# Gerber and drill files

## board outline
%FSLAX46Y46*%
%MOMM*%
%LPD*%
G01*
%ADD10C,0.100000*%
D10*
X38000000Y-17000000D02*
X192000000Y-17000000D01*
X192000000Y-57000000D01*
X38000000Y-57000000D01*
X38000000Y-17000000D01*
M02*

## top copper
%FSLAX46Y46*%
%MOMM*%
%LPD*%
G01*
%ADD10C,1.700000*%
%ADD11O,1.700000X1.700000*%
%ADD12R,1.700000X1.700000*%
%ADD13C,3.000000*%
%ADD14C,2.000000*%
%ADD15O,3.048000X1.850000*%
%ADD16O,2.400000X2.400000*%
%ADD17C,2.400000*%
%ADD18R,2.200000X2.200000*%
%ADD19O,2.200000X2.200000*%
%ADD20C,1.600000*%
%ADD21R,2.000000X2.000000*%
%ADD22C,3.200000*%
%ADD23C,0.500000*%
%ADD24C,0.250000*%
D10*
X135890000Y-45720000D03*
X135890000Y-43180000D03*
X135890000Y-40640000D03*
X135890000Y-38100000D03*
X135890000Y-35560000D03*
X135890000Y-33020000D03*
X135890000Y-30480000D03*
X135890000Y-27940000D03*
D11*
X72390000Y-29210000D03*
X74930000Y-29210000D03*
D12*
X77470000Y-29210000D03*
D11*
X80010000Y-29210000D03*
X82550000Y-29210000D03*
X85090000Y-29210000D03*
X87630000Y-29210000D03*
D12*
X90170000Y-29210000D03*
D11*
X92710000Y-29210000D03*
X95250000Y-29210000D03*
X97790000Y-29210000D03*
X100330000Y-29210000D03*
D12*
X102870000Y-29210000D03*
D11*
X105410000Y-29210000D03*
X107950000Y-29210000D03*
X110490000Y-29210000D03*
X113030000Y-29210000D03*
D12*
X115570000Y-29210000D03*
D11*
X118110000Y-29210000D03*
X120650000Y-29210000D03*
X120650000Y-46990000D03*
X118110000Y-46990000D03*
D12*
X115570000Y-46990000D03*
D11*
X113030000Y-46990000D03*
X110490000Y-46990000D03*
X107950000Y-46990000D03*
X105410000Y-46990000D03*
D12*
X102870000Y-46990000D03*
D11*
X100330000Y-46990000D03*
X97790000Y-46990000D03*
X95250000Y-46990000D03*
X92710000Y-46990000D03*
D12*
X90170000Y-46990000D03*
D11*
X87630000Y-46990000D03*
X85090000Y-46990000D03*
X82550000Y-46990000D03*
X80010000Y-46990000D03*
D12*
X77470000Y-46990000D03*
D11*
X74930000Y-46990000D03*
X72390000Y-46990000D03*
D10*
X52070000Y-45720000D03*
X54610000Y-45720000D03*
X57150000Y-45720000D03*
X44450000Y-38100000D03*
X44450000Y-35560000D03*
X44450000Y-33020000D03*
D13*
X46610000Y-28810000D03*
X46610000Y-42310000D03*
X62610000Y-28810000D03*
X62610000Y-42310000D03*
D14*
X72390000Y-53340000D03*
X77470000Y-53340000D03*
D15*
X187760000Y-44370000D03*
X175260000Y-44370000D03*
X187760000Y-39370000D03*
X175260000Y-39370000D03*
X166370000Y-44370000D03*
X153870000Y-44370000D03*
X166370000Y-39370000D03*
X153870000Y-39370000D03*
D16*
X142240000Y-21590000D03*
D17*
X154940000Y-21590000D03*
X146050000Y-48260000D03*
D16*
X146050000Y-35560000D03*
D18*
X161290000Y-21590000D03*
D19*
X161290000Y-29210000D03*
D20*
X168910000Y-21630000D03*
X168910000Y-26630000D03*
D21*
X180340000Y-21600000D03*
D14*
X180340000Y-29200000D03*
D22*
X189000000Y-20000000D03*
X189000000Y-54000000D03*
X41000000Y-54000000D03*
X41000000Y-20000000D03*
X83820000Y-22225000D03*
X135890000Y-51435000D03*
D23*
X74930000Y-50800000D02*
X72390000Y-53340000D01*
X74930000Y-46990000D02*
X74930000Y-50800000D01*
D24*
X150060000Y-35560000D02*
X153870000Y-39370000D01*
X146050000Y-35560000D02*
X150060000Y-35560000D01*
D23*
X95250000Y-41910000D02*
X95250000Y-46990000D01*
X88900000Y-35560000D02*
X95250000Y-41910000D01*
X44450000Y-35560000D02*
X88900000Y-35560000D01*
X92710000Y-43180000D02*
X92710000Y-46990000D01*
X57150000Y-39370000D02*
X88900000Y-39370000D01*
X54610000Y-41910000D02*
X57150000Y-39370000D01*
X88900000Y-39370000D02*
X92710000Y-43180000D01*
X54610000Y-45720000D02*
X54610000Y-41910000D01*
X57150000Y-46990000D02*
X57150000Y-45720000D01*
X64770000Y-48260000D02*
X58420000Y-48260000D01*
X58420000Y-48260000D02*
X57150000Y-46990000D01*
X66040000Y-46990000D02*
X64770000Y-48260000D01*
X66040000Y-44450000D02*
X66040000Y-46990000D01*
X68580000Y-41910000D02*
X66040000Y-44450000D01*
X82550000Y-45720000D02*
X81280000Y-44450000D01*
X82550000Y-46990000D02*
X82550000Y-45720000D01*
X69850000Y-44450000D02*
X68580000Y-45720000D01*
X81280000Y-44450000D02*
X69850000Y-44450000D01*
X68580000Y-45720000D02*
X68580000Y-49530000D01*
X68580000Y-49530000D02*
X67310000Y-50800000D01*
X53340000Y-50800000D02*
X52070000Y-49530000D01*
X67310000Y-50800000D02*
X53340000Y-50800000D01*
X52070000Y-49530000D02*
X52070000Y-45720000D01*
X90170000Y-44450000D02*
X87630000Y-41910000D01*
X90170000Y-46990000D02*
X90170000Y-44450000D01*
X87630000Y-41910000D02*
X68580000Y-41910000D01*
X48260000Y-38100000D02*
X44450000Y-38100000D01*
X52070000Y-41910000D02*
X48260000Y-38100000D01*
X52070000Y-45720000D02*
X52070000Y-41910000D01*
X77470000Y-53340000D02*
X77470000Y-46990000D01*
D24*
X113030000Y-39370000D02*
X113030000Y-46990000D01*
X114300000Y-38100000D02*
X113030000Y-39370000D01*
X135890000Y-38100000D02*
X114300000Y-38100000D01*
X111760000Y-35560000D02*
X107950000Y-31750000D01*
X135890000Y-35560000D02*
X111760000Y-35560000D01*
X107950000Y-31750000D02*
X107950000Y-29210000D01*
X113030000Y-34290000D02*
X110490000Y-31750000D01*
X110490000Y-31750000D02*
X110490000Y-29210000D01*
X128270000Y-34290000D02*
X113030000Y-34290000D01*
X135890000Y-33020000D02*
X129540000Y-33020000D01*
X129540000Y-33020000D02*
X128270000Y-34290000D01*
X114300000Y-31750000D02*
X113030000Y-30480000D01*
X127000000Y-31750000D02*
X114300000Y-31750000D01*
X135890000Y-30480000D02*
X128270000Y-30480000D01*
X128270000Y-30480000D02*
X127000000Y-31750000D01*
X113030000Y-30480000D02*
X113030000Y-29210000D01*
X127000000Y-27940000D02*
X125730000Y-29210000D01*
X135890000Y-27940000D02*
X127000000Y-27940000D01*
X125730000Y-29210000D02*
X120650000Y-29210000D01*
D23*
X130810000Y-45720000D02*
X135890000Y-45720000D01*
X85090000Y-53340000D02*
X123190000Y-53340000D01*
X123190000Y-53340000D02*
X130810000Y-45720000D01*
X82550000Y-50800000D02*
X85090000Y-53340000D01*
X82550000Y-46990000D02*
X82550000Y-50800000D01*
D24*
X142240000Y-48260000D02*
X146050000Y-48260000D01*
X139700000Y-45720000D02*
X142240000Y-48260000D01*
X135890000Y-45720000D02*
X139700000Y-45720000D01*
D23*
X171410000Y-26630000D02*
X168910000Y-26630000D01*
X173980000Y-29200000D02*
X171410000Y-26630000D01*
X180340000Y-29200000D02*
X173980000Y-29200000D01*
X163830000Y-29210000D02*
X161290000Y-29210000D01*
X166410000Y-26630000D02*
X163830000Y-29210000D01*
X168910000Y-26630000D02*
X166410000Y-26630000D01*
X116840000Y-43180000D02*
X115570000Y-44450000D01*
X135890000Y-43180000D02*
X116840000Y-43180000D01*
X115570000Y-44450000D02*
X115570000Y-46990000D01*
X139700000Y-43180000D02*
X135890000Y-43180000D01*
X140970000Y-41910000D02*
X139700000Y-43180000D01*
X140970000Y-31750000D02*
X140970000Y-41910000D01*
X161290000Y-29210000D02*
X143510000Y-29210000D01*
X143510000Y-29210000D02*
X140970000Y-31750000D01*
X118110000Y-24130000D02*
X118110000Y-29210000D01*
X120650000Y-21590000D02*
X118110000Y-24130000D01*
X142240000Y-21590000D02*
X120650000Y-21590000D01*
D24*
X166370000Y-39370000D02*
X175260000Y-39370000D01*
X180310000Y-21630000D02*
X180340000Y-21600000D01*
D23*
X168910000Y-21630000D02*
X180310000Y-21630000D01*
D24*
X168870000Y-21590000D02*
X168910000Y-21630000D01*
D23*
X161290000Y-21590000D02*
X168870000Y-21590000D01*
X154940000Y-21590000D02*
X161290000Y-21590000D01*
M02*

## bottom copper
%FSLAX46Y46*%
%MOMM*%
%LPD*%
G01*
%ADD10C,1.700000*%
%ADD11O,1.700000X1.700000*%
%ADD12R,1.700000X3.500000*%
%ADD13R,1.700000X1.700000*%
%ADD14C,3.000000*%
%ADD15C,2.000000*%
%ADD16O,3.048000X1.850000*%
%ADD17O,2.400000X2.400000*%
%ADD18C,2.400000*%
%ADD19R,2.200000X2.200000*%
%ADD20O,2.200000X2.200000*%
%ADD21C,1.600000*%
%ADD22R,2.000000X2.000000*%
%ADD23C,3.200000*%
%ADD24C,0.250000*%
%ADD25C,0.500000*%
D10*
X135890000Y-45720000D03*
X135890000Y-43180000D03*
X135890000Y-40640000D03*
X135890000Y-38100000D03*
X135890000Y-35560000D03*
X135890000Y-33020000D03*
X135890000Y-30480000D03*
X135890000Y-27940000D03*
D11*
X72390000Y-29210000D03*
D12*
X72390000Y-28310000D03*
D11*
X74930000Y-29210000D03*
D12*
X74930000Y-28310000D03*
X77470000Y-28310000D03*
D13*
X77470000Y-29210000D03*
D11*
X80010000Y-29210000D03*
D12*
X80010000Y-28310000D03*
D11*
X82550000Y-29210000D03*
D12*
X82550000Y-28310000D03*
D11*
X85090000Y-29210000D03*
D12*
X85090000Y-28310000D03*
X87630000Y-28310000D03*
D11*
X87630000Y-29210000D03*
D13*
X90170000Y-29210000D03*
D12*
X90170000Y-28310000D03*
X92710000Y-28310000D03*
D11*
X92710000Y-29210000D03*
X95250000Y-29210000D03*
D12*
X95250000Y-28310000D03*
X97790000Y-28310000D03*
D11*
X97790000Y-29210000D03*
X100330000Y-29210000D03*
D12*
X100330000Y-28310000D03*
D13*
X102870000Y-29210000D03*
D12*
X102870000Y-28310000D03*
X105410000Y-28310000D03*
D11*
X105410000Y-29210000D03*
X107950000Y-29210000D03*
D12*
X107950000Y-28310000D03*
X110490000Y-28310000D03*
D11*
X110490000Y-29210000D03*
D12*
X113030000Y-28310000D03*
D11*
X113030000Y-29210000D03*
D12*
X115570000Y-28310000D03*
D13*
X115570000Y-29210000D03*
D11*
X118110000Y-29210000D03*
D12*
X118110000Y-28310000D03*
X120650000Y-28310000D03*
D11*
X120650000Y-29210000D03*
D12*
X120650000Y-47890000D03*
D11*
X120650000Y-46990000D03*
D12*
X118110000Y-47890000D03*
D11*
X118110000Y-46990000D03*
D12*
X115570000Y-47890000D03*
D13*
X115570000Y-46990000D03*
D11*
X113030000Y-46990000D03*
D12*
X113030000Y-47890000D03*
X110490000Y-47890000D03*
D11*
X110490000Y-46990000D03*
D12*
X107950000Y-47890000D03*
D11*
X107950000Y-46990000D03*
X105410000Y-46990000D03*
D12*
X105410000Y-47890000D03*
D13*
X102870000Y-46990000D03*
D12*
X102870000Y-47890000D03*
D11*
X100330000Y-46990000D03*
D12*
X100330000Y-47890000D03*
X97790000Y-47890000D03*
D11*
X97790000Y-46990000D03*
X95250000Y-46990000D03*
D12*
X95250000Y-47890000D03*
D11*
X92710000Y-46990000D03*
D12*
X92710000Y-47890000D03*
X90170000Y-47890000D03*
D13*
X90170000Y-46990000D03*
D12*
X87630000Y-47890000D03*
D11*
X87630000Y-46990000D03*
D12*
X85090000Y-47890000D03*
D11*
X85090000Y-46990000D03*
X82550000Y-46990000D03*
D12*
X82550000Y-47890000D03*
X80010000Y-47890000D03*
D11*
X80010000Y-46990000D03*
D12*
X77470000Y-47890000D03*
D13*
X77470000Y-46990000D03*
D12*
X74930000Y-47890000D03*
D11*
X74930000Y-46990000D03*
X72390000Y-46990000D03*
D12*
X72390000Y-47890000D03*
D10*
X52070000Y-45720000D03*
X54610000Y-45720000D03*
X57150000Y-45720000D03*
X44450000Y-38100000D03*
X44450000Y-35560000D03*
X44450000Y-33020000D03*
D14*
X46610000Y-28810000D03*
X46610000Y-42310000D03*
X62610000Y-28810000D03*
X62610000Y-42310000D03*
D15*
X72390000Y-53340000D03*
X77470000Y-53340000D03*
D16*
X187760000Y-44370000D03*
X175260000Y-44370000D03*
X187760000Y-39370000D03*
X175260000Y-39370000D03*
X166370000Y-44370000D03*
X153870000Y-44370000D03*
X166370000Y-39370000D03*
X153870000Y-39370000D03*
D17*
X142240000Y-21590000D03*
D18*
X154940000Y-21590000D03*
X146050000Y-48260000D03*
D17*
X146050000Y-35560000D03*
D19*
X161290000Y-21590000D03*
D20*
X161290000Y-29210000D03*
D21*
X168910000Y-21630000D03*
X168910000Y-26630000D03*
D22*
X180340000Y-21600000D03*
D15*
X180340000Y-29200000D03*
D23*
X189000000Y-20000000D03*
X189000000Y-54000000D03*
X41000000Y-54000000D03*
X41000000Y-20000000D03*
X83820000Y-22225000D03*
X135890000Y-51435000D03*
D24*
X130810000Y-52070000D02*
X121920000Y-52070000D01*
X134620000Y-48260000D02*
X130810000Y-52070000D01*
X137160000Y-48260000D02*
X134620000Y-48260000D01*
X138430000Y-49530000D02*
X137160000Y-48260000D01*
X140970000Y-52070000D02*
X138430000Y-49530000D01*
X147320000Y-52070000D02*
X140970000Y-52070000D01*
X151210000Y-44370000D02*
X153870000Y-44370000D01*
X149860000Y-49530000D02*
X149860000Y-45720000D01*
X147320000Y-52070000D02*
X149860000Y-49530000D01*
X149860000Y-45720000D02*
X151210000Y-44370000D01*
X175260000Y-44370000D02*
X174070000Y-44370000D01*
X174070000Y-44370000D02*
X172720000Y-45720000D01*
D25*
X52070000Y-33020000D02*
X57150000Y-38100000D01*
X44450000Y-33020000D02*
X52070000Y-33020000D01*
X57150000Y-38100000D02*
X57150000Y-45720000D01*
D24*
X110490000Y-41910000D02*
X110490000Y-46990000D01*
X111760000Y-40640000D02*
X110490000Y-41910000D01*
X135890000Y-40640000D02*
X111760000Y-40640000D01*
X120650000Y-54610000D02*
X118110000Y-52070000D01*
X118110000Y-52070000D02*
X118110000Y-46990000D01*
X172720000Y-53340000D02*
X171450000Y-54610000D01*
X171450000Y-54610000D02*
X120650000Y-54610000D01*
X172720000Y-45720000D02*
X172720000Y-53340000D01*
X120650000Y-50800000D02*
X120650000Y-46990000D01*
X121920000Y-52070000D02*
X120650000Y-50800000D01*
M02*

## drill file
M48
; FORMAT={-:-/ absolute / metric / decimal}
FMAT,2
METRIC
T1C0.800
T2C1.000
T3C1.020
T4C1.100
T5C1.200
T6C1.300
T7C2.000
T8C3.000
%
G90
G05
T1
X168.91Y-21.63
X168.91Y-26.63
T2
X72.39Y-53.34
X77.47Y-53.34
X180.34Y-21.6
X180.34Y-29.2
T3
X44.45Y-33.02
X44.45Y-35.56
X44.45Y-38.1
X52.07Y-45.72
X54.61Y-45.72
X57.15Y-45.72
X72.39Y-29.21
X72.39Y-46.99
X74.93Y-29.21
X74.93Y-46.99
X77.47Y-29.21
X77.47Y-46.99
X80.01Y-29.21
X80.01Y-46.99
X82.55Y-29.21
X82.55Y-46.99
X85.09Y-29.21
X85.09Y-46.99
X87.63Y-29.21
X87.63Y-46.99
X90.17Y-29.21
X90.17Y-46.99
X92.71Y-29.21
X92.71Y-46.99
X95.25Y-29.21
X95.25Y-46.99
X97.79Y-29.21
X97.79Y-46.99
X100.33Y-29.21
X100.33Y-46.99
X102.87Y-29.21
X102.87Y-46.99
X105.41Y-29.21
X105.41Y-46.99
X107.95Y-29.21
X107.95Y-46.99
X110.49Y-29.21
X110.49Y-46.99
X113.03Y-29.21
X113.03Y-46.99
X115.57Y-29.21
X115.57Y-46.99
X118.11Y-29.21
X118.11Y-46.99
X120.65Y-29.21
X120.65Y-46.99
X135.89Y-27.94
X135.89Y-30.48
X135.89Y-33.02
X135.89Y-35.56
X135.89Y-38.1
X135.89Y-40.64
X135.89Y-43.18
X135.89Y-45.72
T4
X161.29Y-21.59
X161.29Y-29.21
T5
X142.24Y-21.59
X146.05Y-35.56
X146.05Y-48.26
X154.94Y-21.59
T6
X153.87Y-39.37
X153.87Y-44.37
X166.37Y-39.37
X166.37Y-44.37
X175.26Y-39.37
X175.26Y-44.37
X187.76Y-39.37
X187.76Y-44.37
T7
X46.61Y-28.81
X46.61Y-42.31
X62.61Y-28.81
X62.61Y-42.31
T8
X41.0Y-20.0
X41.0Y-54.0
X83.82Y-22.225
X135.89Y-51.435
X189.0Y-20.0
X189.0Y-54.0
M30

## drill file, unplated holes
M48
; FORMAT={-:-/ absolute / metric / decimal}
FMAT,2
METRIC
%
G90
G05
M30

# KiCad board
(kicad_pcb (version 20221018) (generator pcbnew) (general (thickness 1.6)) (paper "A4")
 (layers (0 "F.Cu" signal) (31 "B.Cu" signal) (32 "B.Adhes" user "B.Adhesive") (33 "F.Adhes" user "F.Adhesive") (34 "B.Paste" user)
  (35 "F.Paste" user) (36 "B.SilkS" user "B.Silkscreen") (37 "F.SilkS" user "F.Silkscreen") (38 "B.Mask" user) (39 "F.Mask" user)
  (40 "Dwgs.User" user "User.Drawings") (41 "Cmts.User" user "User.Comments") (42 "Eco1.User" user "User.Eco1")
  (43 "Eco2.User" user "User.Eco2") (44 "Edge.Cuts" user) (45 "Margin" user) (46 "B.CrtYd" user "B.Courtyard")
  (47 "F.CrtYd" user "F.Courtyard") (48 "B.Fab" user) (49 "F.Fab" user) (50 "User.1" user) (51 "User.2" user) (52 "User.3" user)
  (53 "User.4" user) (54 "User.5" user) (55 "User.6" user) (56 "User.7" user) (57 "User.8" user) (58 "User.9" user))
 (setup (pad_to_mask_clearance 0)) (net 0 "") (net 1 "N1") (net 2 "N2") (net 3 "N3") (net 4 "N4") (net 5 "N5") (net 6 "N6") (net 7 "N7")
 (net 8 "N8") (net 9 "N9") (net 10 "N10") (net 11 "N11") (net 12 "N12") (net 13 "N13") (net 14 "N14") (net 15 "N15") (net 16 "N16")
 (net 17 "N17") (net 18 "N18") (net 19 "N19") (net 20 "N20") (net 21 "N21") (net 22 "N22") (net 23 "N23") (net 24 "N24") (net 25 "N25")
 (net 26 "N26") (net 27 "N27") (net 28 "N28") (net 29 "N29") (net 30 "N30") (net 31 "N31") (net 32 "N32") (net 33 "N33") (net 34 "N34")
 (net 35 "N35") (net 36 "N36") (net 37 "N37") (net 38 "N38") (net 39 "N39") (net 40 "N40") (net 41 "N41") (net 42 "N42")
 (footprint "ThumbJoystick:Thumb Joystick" (layer "F.Cu") (at 54.61 35.56)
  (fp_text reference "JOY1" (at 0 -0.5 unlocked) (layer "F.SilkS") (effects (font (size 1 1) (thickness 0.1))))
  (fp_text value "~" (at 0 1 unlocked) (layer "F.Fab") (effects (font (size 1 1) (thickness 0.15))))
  (pad "1" thru_hole circle (at -2.54 10.16) (size 1.7 1.7) (drill 1.02) (layers "*.Cu" "*.Mask") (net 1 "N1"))
  (pad "2" thru_hole circle (at 0 10.16) (size 1.7 1.7) (drill 1.02) (layers "*.Cu" "*.Mask") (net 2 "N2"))
  (pad "3" thru_hole circle (at 2.54 10.16) (size 1.7 1.7) (drill 1.02) (layers "*.Cu" "*.Mask") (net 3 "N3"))
  (pad "4" thru_hole circle (at -10.16 2.54) (size 1.7 1.7) (drill 1.02) (layers "*.Cu" "*.Mask") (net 1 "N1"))
  (pad "5" thru_hole circle (at -10.16 0) (size 1.7 1.7) (drill 1.02) (layers "*.Cu" "*.Mask") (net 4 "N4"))
  (pad "6" thru_hole circle (at -10.16 -2.54) (size 1.7 1.7) (drill 1.02) (layers "*.Cu" "*.Mask") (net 3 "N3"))
  (pad "8" thru_hole circle (at -8 -6.75) (size 3 3) (drill 2) (layers "*.Cu" "*.Mask"))
  (pad "8" thru_hole circle (at -8 6.75) (size 3 3) (drill 2) (layers "*.Cu" "*.Mask"))
  (pad "8" thru_hole circle (at 8 -6.75) (size 3 3) (drill 2) (layers "*.Cu" "*.Mask"))
  (pad "8" thru_hole circle (at 8 6.75) (size 3 3) (drill 2) (layers "*.Cu" "*.Mask")))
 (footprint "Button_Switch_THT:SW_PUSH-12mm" (layer "F.Cu") (at 153.87 39.37)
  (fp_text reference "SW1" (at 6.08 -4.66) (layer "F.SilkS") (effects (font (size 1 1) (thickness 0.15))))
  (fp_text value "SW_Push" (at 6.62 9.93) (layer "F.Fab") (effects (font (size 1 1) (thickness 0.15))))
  (pad "1" thru_hole oval (at 0 0) (size 3.048 1.85) (drill 1.3) (layers "*.Cu" "*.Mask") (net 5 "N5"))
  (pad "1" thru_hole oval (at 12.5 0) (size 3.048 1.85) (drill 1.3) (layers "*.Cu" "*.Mask") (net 5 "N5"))
  (pad "2" thru_hole oval (at 0 5) (size 3.048 1.85) (drill 1.3) (layers "*.Cu" "*.Mask") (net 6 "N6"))
  (pad "2" thru_hole oval (at 12.5 5) (size 3.048 1.85) (drill 1.3) (layers "*.Cu" "*.Mask") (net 6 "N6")))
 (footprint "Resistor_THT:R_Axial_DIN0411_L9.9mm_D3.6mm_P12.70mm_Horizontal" (layer "F.Cu") (at 154.94 21.59 180)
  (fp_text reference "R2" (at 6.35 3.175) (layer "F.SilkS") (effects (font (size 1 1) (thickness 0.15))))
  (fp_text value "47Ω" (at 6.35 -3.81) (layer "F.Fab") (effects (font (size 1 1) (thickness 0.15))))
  (pad "1" thru_hole circle (at 0 0 180) (size 2.4 2.4) (drill 1.2) (layers "*.Cu" "*.Mask") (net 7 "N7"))
  (pad "2" thru_hole oval (at 12.7 0 180) (size 2.4 2.4) (drill 1.2) (layers "*.Cu" "*.Mask") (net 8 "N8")))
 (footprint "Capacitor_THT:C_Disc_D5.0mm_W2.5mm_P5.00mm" (layer "F.Cu") (at 168.91 21.63 -90)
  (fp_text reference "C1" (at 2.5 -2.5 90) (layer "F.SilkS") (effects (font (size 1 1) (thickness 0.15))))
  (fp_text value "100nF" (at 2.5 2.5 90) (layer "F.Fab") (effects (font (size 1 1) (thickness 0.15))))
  (pad "1" thru_hole circle (at 0 0 270) (size 1.6 1.6) (drill 0.8) (layers "*.Cu" "*.Mask") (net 7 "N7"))
  (pad "2" thru_hole circle (at 5 0 270) (size 1.6 1.6) (drill 0.8) (layers "*.Cu" "*.Mask") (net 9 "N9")))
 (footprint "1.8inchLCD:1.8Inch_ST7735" (layer "F.Cu") (at 135.89 36.83)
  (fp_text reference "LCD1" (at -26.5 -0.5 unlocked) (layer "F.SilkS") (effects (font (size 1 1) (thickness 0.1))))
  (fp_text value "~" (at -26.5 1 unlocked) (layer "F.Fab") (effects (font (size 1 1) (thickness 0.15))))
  (pad "1" thru_hole circle (at 0 8.89) (size 1.7 1.7) (drill 1.02) (layers "*.Cu" "*.Mask") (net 1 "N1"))
  (pad "2" thru_hole circle (at 0 6.35) (size 1.7 1.7) (drill 1.02) (layers "*.Cu" "*.Mask") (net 9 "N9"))
  (pad "3" thru_hole circle (at 0 3.81) (size 1.7 1.7) (drill 1.02) (layers "*.Cu" "*.Mask") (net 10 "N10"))
  (pad "4" thru_hole circle (at 0 1.27) (size 1.7 1.7) (drill 1.02) (layers "*.Cu" "*.Mask") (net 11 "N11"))
  (pad "5" thru_hole circle (at 0 -1.27) (size 1.7 1.7) (drill 1.02) (layers "*.Cu" "*.Mask") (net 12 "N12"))
  (pad "6" thru_hole circle (at 0 -3.81) (size 1.7 1.7) (drill 1.02) (layers "*.Cu" "*.Mask") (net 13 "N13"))
  (pad "7" thru_hole circle (at 0 -6.35) (size 1.7 1.7) (drill 1.02) (layers "*.Cu" "*.Mask") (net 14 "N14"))
  (pad "8" thru_hole circle (at 0 -8.89) (size 1.7 1.7) (drill 1.02) (layers "*.Cu" "*.Mask") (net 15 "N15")))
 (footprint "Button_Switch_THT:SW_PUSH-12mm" (layer "F.Cu") (at 175.26 39.37)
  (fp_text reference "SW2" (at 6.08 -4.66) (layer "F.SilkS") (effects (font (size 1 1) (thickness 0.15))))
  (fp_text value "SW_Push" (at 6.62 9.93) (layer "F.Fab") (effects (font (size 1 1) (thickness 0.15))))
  (pad "1" thru_hole oval (at 0 0) (size 3.048 1.85) (drill 1.3) (layers "*.Cu" "*.Mask") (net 5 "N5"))
  (pad "1" thru_hole oval (at 12.5 0) (size 3.048 1.85) (drill 1.3) (layers "*.Cu" "*.Mask") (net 5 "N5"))
  (pad "2" thru_hole oval (at 0 5) (size 3.048 1.85) (drill 1.3) (layers "*.Cu" "*.Mask") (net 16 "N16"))
  (pad "2" thru_hole oval (at 12.5 5) (size 3.048 1.85) (drill 1.3) (layers "*.Cu" "*.Mask") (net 16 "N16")))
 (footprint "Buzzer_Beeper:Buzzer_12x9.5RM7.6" (layer "F.Cu") (at 180.34 21.6 -90)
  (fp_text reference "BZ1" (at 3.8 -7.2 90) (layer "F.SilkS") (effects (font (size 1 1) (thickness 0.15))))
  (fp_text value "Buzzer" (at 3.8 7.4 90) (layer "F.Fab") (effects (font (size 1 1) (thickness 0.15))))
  (pad "1" thru_hole rect (at 0 0 270) (size 2 2) (drill 1) (layers "*.Cu" "*.Mask") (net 7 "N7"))
  (pad "2" thru_hole circle (at 7.6 0 270) (size 2 2) (drill 1) (layers "*.Cu" "*.Mask") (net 9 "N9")))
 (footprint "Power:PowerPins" (layer "F.Cu") (at 74.93 53.34)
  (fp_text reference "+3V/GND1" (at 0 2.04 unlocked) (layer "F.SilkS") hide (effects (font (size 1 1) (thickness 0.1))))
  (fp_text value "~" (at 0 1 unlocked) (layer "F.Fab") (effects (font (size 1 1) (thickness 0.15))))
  (pad "1" thru_hole circle (at -2.54 0) (size 2 2) (drill 1) (layers "*.Cu" "*.Mask") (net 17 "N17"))
  (pad "2" thru_hole circle (at 2.54 0) (size 2 2) (drill 1) (layers "*.Cu" "*.Mask") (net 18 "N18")))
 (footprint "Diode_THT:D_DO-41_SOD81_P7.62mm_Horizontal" (layer "F.Cu") (at 161.29 21.59 -90)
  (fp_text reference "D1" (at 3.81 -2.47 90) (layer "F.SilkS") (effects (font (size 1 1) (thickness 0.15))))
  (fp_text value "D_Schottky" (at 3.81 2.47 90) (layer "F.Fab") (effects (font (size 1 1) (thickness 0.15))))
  (pad "1" thru_hole rect (at 0 0 270) (size 2.2 2.2) (drill 1.1) (layers "*.Cu" "*.Mask") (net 7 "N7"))
  (pad "2" thru_hole oval (at 7.62 0 270) (size 2.2 2.2) (drill 1.1) (layers "*.Cu" "*.Mask") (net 9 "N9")))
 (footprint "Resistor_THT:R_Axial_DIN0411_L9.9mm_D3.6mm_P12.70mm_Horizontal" (layer "F.Cu") (at 146.05 48.26 90)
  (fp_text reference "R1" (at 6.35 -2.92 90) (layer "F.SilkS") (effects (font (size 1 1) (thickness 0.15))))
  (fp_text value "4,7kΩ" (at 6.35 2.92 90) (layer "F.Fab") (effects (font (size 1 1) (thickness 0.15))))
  (pad "1" thru_hole circle (at 0 0 90) (size 2.4 2.4) (drill 1.2) (layers "*.Cu" "*.Mask") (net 1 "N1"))
  (pad "2" thru_hole oval (at 12.7 0 90) (size 2.4 2.4) (drill 1.2) (layers "*.Cu" "*.Mask") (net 5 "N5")))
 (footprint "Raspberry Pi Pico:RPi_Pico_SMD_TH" (layer "B.Cu") (at 96.52 38.1 -90)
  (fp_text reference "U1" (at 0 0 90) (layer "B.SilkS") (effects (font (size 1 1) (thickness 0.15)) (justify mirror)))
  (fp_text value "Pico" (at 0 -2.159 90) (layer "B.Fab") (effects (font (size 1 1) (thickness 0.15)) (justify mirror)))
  (pad "1" thru_hole oval (at -8.89 24.13 270) (size 1.7 1.7) (drill 1.02) (layers "*.Cu" "*.Mask") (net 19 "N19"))
  (pad "1" smd rect (at -8.89 24.13 270) (size 3.5 1.7) (drill (offset -0.9 0)) (layers "B.Cu" "B.Mask") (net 19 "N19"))
  (pad "2" thru_hole oval (at -8.89 21.59 270) (size 1.7 1.7) (drill 1.02) (layers "*.Cu" "*.Mask") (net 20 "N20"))
  (pad "2" smd rect (at -8.89 21.59 270) (size 3.5 1.7) (drill (offset -0.9 0)) (layers "B.Cu" "B.Mask") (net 20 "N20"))
  (pad "3" thru_hole rect (at -8.89 19.05 270) (size 1.7 1.7) (drill 1.02) (layers "*.Cu" "*.Mask") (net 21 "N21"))
  (pad "3" smd rect (at -8.89 19.05 270) (size 3.5 1.7) (drill (offset -0.9 0)) (layers "B.Cu" "B.Mask") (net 21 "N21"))
  (pad "4" thru_hole oval (at -8.89 16.51 270) (size 1.7 1.7) (drill 1.02) (layers "*.Cu" "*.Mask") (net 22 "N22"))
  (pad "4" smd rect (at -8.89 16.51 270) (size 3.5 1.7) (drill (offset -0.9 0)) (layers "B.Cu" "B.Mask") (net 22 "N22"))
  (pad "5" thru_hole oval (at -8.89 13.97 270) (size 1.7 1.7) (drill 1.02) (layers "*.Cu" "*.Mask") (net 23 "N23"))
  (pad "5" smd rect (at -8.89 13.97 270) (size 3.5 1.7) (drill (offset -0.9 0)) (layers "B.Cu" "B.Mask") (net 23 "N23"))
  (pad "6" thru_hole oval (at -8.89 11.43 270) (size 1.7 1.7) (drill 1.02) (layers "*.Cu" "*.Mask") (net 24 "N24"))
  (pad "6" smd rect (at -8.89 11.43 270) (size 3.5 1.7) (drill (offset -0.9 0)) (layers "B.Cu" "B.Mask") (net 24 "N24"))
  (pad "7" thru_hole oval (at -8.89 8.89 270) (size 1.7 1.7) (drill 1.02) (layers "*.Cu" "*.Mask") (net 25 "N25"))
  (pad "7" smd rect (at -8.89 8.89 270) (size 3.5 1.7) (drill (offset -0.9 0)) (layers "B.Cu" "B.Mask") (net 25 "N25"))
  (pad "8" thru_hole rect (at -8.89 6.35 270) (size 1.7 1.7) (drill 1.02) (layers "*.Cu" "*.Mask") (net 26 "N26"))
  (pad "8" smd rect (at -8.89 6.35 270) (size 3.5 1.7) (drill (offset -0.9 0)) (layers "B.Cu" "B.Mask") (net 26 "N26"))
  (pad "9" thru_hole oval (at -8.89 3.81 270) (size 1.7 1.7) (drill 1.02) (layers "*.Cu" "*.Mask") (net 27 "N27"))
  (pad "9" smd rect (at -8.89 3.81 270) (size 3.5 1.7) (drill (offset -0.9 0)) (layers "B.Cu" "B.Mask") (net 27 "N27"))
  (pad "10" thru_hole oval (at -8.89 1.27 270) (size 1.7 1.7) (drill 1.02) (layers "*.Cu" "*.Mask") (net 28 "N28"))
  (pad "10" smd rect (at -8.89 1.27 270) (size 3.5 1.7) (drill (offset -0.9 0)) (layers "B.Cu" "B.Mask") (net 28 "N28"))
  (pad "11" thru_hole oval (at -8.89 -1.27 270) (size 1.7 1.7) (drill 1.02) (layers "*.Cu" "*.Mask") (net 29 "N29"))
  (pad "11" smd rect (at -8.89 -1.27 270) (size 3.5 1.7) (drill (offset -0.9 0)) (layers "B.Cu" "B.Mask") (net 29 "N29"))
  (pad "12" thru_hole oval (at -8.89 -3.81 270) (size 1.7 1.7) (drill 1.02) (layers "*.Cu" "*.Mask") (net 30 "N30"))
  (pad "12" smd rect (at -8.89 -3.81 270) (size 3.5 1.7) (drill (offset -0.9 0)) (layers "B.Cu" "B.Mask") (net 30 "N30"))
  (pad "13" thru_hole rect (at -8.89 -6.35 270) (size 1.7 1.7) (drill 1.02) (layers "*.Cu" "*.Mask") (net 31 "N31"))
  (pad "13" smd rect (at -8.89 -6.35 270) (size 3.5 1.7) (drill (offset -0.9 0)) (layers "B.Cu" "B.Mask") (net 31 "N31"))
  (pad "14" thru_hole oval (at -8.89 -8.89 270) (size 1.7 1.7) (drill 1.02) (layers "*.Cu" "*.Mask") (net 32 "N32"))
  (pad "14" smd rect (at -8.89 -8.89 270) (size 3.5 1.7) (drill (offset -0.9 0)) (layers "B.Cu" "B.Mask") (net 32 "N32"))
  (pad "15" thru_hole oval (at -8.89 -11.43 270) (size 1.7 1.7) (drill 1.02) (layers "*.Cu" "*.Mask") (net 12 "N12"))
  (pad "15" smd rect (at -8.89 -11.43 270) (size 3.5 1.7) (drill (offset -0.9 0)) (layers "B.Cu" "B.Mask") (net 12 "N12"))
  (pad "16" thru_hole oval (at -8.89 -13.97 270) (size 1.7 1.7) (drill 1.02) (layers "*.Cu" "*.Mask") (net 13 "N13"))
  (pad "16" smd rect (at -8.89 -13.97 270) (size 3.5 1.7) (drill (offset -0.9 0)) (layers "B.Cu" "B.Mask") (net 13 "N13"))
  (pad "17" thru_hole oval (at -8.89 -16.51 270) (size 1.7 1.7) (drill 1.02) (layers "*.Cu" "*.Mask") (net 14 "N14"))
  (pad "17" smd rect (at -8.89 -16.51 270) (size 3.5 1.7) (drill (offset -0.9 0)) (layers "B.Cu" "B.Mask") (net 14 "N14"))
  (pad "18" thru_hole rect (at -8.89 -19.05 270) (size 1.7 1.7) (drill 1.02) (layers "*.Cu" "*.Mask") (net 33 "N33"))
  (pad "18" smd rect (at -8.89 -19.05 270) (size 3.5 1.7) (drill (offset -0.9 0)) (layers "B.Cu" "B.Mask") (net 33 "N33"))
  (pad "19" thru_hole oval (at -8.89 -21.59 270) (size 1.7 1.7) (drill 1.02) (layers "*.Cu" "*.Mask") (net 8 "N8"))
  (pad "19" smd rect (at -8.89 -21.59 270) (size 3.5 1.7) (drill (offset -0.9 0)) (layers "B.Cu" "B.Mask") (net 8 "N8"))
  (pad "20" thru_hole oval (at -8.89 -24.13 270) (size 1.7 1.7) (drill 1.02) (layers "*.Cu" "*.Mask") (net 15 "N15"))
  (pad "20" smd rect (at -8.89 -24.13 270) (size 3.5 1.7) (drill (offset -0.9 0)) (layers "B.Cu" "B.Mask") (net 15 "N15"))
  (pad "21" thru_hole oval (at 8.89 -24.13 270) (size 1.7 1.7) (drill 1.02) (layers "*.Cu" "*.Mask") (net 6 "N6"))
  (pad "21" smd rect (at 8.89 -24.13 270) (size 3.5 1.7) (drill (offset 0.9 0)) (layers "B.Cu" "B.Mask") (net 6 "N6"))
  (pad "22" thru_hole oval (at 8.89 -21.59 270) (size 1.7 1.7) (drill 1.02) (layers "*.Cu" "*.Mask") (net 16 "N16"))
  (pad "22" smd rect (at 8.89 -21.59 270) (size 3.5 1.7) (drill (offset 0.9 0)) (layers "B.Cu" "B.Mask") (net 16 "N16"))
  (pad "23" thru_hole rect (at 8.89 -19.05 270) (size 1.7 1.7) (drill 1.02) (layers "*.Cu" "*.Mask") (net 9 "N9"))
  (pad "23" smd rect (at 8.89 -19.05 270) (size 3.5 1.7) (drill (offset 0.9 0)) (layers "B.Cu" "B.Mask") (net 9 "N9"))
  (pad "24" thru_hole oval (at 8.89 -16.51 270) (size 1.7 1.7) (drill 1.02) (layers "*.Cu" "*.Mask") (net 11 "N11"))
  (pad "24" smd rect (at 8.89 -16.51 270) (size 3.5 1.7) (drill (offset 0.9 0)) (layers "B.Cu" "B.Mask") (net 11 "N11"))
  (pad "25" thru_hole oval (at 8.89 -13.97 270) (size 1.7 1.7) (drill 1.02) (layers "*.Cu" "*.Mask") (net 10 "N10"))
  (pad "25" smd rect (at 8.89 -13.97 270) (size 3.5 1.7) (drill (offset 0.9 0)) (layers "B.Cu" "B.Mask") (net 10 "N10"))
  (pad "26" thru_hole oval (at 8.89 -11.43 270) (size 1.7 1.7) (drill 1.02) (layers "*.Cu" "*.Mask") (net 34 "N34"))
  (pad "26" smd rect (at 8.89 -11.43 270) (size 3.5 1.7) (drill (offset 0.9 0)) (layers "B.Cu" "B.Mask") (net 34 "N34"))
  (pad "27" thru_hole oval (at 8.89 -8.89 270) (size 1.7 1.7) (drill 1.02) (layers "*.Cu" "*.Mask") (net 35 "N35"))
  (pad "27" smd rect (at 8.89 -8.89 270) (size 3.5 1.7) (drill (offset 0.9 0)) (layers "B.Cu" "B.Mask") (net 35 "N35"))
  (pad "28" thru_hole rect (at 8.89 -6.35 270) (size 1.7 1.7) (drill 1.02) (layers "*.Cu" "*.Mask") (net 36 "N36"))
  (pad "28" smd rect (at 8.89 -6.35 270) (size 3.5 1.7) (drill (offset 0.9 0)) (layers "B.Cu" "B.Mask") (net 36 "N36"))
  (pad "29" thru_hole oval (at 8.89 -3.81 270) (size 1.7 1.7) (drill 1.02) (layers "*.Cu" "*.Mask") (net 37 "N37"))
  (pad "29" smd rect (at 8.89 -3.81 270) (size 3.5 1.7) (drill (offset 0.9 0)) (layers "B.Cu" "B.Mask") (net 37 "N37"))
  (pad "30" thru_hole oval (at 8.89 -1.27 270) (size 1.7 1.7) (drill 1.02) (layers "*.Cu" "*.Mask") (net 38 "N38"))
  (pad "30" smd rect (at 8.89 -1.27 270) (size 3.5 1.7) (drill (offset 0.9 0)) (layers "B.Cu" "B.Mask") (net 38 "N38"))
  (pad "31" thru_hole oval (at 8.89 1.27 270) (size 1.7 1.7) (drill 1.02) (layers "*.Cu" "*.Mask") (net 4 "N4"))
  (pad "31" smd rect (at 8.89 1.27 270) (size 3.5 1.7) (drill (offset 0.9 0)) (layers "B.Cu" "B.Mask") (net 4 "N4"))
  (pad "32" thru_hole oval (at 8.89 3.81 270) (size 1.7 1.7) (drill 1.02) (layers "*.Cu" "*.Mask") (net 2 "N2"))
  (pad "32" smd rect (at 8.89 3.81 270) (size 3.5 1.7) (drill (offset 0.9 0)) (layers "B.Cu" "B.Mask") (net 2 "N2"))
  (pad "33" thru_hole rect (at 8.89 6.35 270) (size 1.7 1.7) (drill 1.02) (layers "*.Cu" "*.Mask") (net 3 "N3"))
  (pad "33" smd rect (at 8.89 6.35 270) (size 3.5 1.7) (drill (offset 0.9 0)) (layers "B.Cu" "B.Mask") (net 3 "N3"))
  (pad "34" thru_hole oval (at 8.89 8.89 270) (size 1.7 1.7) (drill 1.02) (layers "*.Cu" "*.Mask") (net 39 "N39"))
  (pad "34" smd rect (at 8.89 8.89 270) (size 3.5 1.7) (drill (offset 0.9 0)) (layers "B.Cu" "B.Mask") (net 39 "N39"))
  (pad "35" thru_hole oval (at 8.89 11.43 270) (size 1.7 1.7) (drill 1.02) (layers "*.Cu" "*.Mask") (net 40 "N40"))
  (pad "35" smd rect (at 8.89 11.43 270) (size 3.5 1.7) (drill (offset 0.9 0)) (layers "B.Cu" "B.Mask") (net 40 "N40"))
  (pad "36" thru_hole oval (at 8.89 13.97 270) (size 1.7 1.7) (drill 1.02) (layers "*.Cu" "*.Mask") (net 1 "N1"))
  (pad "36" smd rect (at 8.89 13.97 270) (size 3.5 1.7) (drill (offset 0.9 0)) (layers "B.Cu" "B.Mask") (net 1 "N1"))
  (pad "37" thru_hole oval (at 8.89 16.51 270) (size 1.7 1.7) (drill 1.02) (layers "*.Cu" "*.Mask") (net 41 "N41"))
  (pad "37" smd rect (at 8.89 16.51 270) (size 3.5 1.7) (drill (offset 0.9 0)) (layers "B.Cu" "B.Mask") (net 41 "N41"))
  (pad "38" thru_hole rect (at 8.89 19.05 270) (size 1.7 1.7) (drill 1.02) (layers "*.Cu" "*.Mask") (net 18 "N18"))
  (pad "38" smd rect (at 8.89 19.05 270) (size 3.5 1.7) (drill (offset 0.9 0)) (layers "B.Cu" "B.Mask") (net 18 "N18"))
  (pad "39" thru_hole oval (at 8.89 21.59 270) (size 1.7 1.7) (drill 1.02) (layers "*.Cu" "*.Mask") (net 17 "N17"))
  (pad "39" smd rect (at 8.89 21.59 270) (size 3.5 1.7) (drill (offset 0.9 0)) (layers "B.Cu" "B.Mask") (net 17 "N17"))
  (pad "40" thru_hole oval (at 8.89 24.13 270) (size 1.7 1.7) (drill 1.02) (layers "*.Cu" "*.Mask") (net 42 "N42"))
  (pad "40" smd rect (at 8.89 24.13 270) (size 3.5 1.7) (drill (offset 0.9 0)) (layers "B.Cu" "B.Mask") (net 42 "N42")))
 (gr_rect (start 38 17) (end 192 57) (stroke (width 0.1) (type default)) (fill none) (layer "Edge.Cuts"))
 (via (at 135.89 51.435) (size 3.2) (drill 3) (layers "F.Cu" "B.Cu") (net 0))
 (via (at 41 54) (size 3.2) (drill 3) (layers "F.Cu" "B.Cu") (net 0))
 (via (at 189 54) (size 3.2) (drill 3) (layers "F.Cu" "B.Cu") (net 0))
 (via (at 189 20) (size 3.2) (drill 3) (layers "F.Cu" "B.Cu") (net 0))
 (via (at 41 20) (size 3.2) (drill 3) (layers "F.Cu" "B.Cu") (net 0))
 (via (at 83.82 22.225) (size 3.2) (drill 3) (layers "F.Cu" "B.Cu") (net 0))
 (segment (start 168.87 21.59) (end 168.91 21.63) (width 0.25) (layer "F.Cu") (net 7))
 (segment (start 168.91 21.63) (end 180.31 21.63) (width 0.5) (layer "F.Cu") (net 7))
 (segment (start 161.29 21.59) (end 168.87 21.59) (width 0.5) (layer "F.Cu") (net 7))
 (segment (start 180.31 21.63) (end 180.34 21.6) (width 0.25) (layer "F.Cu") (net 7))
 (segment (start 154.94 21.59) (end 161.29 21.59) (width 0.5) (layer "F.Cu") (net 7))
 (segment (start 140.97 41.91) (end 139.7 43.18) (width 0.5) (layer "F.Cu") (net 9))
 (segment (start 173.98 29.2) (end 171.41 26.63) (width 0.5) (layer "F.Cu") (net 9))
 (segment (start 168.91 26.63) (end 166.41 26.63) (width 0.5) (layer "F.Cu") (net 9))
 (segment (start 143.51 29.21) (end 140.97 31.75) (width 0.5) (layer "F.Cu") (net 9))
 (segment (start 161.29 29.21) (end 143.51 29.21) (width 0.5) (layer "F.Cu") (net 9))
 (segment (start 171.41 26.63) (end 168.91 26.63) (width 0.5) (layer "F.Cu") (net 9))
 (segment (start 163.83 29.21) (end 161.29 29.21) (width 0.5) (layer "F.Cu") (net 9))
 (segment (start 135.89 43.18) (end 116.84 43.18) (width 0.5) (layer "F.Cu") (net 9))
 (segment (start 116.84 43.18) (end 115.57 44.45) (width 0.5) (layer "F.Cu") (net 9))
 (segment (start 166.41 26.63) (end 163.83 29.21) (width 0.5) (layer "F.Cu") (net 9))
 (segment (start 140.97 31.75) (end 140.97 41.91) (width 0.5) (layer "F.Cu") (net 9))
 (segment (start 139.7 43.18) (end 135.89 43.18) (width 0.5) (layer "F.Cu") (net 9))
 (segment (start 115.57 44.45) (end 115.57 46.99) (width 0.5) (layer "F.Cu") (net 9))
 (segment (start 180.34 29.2) (end 173.98 29.2) (width 0.5) (layer "F.Cu") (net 9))
 (segment (start 68.58 49.53) (end 67.31 50.8) (width 0.5) (layer "F.Cu") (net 1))
 (segment (start 82.55 50.8) (end 85.09 53.34) (width 0.5) (layer "F.Cu") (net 1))
 (segment (start 52.07 45.72) (end 52.07 41.91) (width 0.5) (layer "F.Cu") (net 1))
 (segment (start 68.58 45.72) (end 68.58 49.53) (width 0.5) (layer "F.Cu") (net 1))
 (segment (start 85.09 53.34) (end 123.19 53.34) (width 0.5) (layer "F.Cu") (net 1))
 (segment (start 135.89 45.72) (end 139.7 45.72) (width 0.25) (layer "F.Cu") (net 1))
 (segment (start 82.55 45.72) (end 81.28 44.45) (width 0.5) (layer "F.Cu") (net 1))
 (segment (start 67.31 50.8) (end 53.34 50.8) (width 0.5) (layer "F.Cu") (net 1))
 (segment (start 52.07 41.91) (end 48.26 38.1) (width 0.5) (layer "F.Cu") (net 1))
 (segment (start 82.55 46.99) (end 82.55 45.72) (width 0.5) (layer "F.Cu") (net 1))
 (segment (start 48.26 38.1) (end 44.45 38.1) (width 0.5) (layer "F.Cu") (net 1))
 (segment (start 53.34 50.8) (end 52.07 49.53) (width 0.5) (layer "F.Cu") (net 1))
 (segment (start 139.7 45.72) (end 142.24 48.26) (width 0.25) (layer "F.Cu") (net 1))
 (segment (start 123.19 53.34) (end 130.81 45.72) (width 0.5) (layer "F.Cu") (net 1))
 (segment (start 52.07 49.53) (end 52.07 45.72) (width 0.5) (layer "F.Cu") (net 1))
 (segment (start 69.85 44.45) (end 68.58 45.72) (width 0.5) (layer "F.Cu") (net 1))
 (segment (start 130.81 45.72) (end 135.89 45.72) (width 0.5) (layer "F.Cu") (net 1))
 (segment (start 142.24 48.26) (end 146.05 48.26) (width 0.25) (layer "F.Cu") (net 1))
 (segment (start 82.55 46.99) (end 82.55 50.8) (width 0.5) (layer "F.Cu") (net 1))
 (segment (start 81.28 44.45) (end 69.85 44.45) (width 0.5) (layer "F.Cu") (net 1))
 (segment (start 95.25 41.91) (end 95.25 46.99) (width 0.5) (layer "F.Cu") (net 4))
 (segment (start 44.45 35.56) (end 88.9 35.56) (width 0.5) (layer "F.Cu") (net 4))
 (segment (start 88.9 35.56) (end 95.25 41.91) (width 0.5) (layer "F.Cu") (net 4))
 (segment (start 68.58 41.91) (end 66.04 44.45) (width 0.5) (layer "F.Cu") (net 3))
 (segment (start 64.77 48.26) (end 58.42 48.26) (width 0.5) (layer "F.Cu") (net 3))
 (segment (start 57.15 46.99) (end 57.15 45.72) (width 0.5) (layer "F.Cu") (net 3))
 (segment (start 90.17 44.45) (end 87.63 41.91) (width 0.5) (layer "F.Cu") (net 3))
 (segment (start 87.63 41.91) (end 68.58 41.91) (width 0.5) (layer "F.Cu") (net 3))
 (segment (start 66.04 44.45) (end 66.04 46.99) (width 0.5) (layer "F.Cu") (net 3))
 (segment (start 58.42 48.26) (end 57.15 46.99) (width 0.5) (layer "F.Cu") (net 3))
 (segment (start 66.04 46.99) (end 64.77 48.26) (width 0.5) (layer "F.Cu") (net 3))
 (segment (start 90.17 46.99) (end 90.17 44.45) (width 0.5) (layer "F.Cu") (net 3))
 (segment (start 52.07 33.02) (end 57.15 38.1) (width 0.5) (layer "B.Cu") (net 3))
 (segment (start 57.15 38.1) (end 57.15 45.72) (width 0.5) (layer "B.Cu") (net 3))
 (segment (start 44.45 33.02) (end 52.07 33.02) (width 0.5) (layer "B.Cu") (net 3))
 (segment (start 57.15 39.37) (end 88.9 39.37) (width 0.5) (layer "F.Cu") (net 2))
 (segment (start 88.9 39.37) (end 92.71 43.18) (width 0.5) (layer "F.Cu") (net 2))
 (segment (start 54.61 41.91) (end 57.15 39.37) (width 0.5) (layer "F.Cu") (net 2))
 (segment (start 54.61 45.72) (end 54.61 41.91) (width 0.5) (layer "F.Cu") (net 2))
 (segment (start 92.71 43.18) (end 92.71 46.99) (width 0.5) (layer "F.Cu") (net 2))
 (segment (start 146.05 35.56) (end 150.06 35.56) (width 0.25) (layer "F.Cu") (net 5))
 (segment (start 166.37 39.37) (end 175.26 39.37) (width 0.25) (layer "F.Cu") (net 5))
 (segment (start 150.06 35.56) (end 153.87 39.37) (width 0.25) (layer "F.Cu") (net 5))
 (segment (start 142.24 21.59) (end 120.65 21.59) (width 0.5) (layer "F.Cu") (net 8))
 (segment (start 118.11 24.13) (end 118.11 29.21) (width 0.5) (layer "F.Cu") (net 8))
 (segment (start 120.65 21.59) (end 118.11 24.13) (width 0.5) (layer "F.Cu") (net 8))
 (segment (start 174.07 44.37) (end 172.72 45.72) (width 0.25) (layer "B.Cu") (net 16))
 (segment (start 120.65 54.61) (end 118.11 52.07) (width 0.25) (layer "B.Cu") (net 16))
 (segment (start 172.72 53.34) (end 171.45 54.61) (width 0.25) (layer "B.Cu") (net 16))
 (segment (start 171.45 54.61) (end 120.65 54.61) (width 0.25) (layer "B.Cu") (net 16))
 (segment (start 172.72 45.72) (end 172.72 53.34) (width 0.25) (layer "B.Cu") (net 16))
 (segment (start 175.26 44.37) (end 174.07 44.37) (width 0.25) (layer "B.Cu") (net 16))
 (segment (start 118.11 52.07) (end 118.11 46.99) (width 0.25) (layer "B.Cu") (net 16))
 (segment (start 134.62 48.26) (end 130.81 52.07) (width 0.25) (layer "B.Cu") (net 6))
 (segment (start 151.21 44.37) (end 153.87 44.37) (width 0.25) (layer "B.Cu") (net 6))
 (segment (start 137.16 48.26) (end 134.62 48.26) (width 0.25) (layer "B.Cu") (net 6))
 (segment (start 147.32 52.07) (end 149.86 49.53) (width 0.25) (layer "B.Cu") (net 6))
 (segment (start 147.32 52.07) (end 140.97 52.07) (width 0.25) (layer "B.Cu") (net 6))
 (segment (start 120.65 50.8) (end 120.65 46.99) (width 0.25) (layer "B.Cu") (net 6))
 (segment (start 121.92 52.07) (end 120.65 50.8) (width 0.25) (layer "B.Cu") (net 6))
 (segment (start 138.43 49.53) (end 137.16 48.26) (width 0.25) (layer "B.Cu") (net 6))
 (segment (start 130.81 52.07) (end 121.92 52.07) (width 0.25) (layer "B.Cu") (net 6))
 (segment (start 149.86 49.53) (end 149.86 45.72) (width 0.25) (layer "B.Cu") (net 6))
 (segment (start 140.97 52.07) (end 138.43 49.53) (width 0.25) (layer "B.Cu") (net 6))
 (segment (start 149.86 45.72) (end 151.21 44.37) (width 0.25) (layer "B.Cu") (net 6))
 (segment (start 135.89 33.02) (end 129.54 33.02) (width 0.25) (layer "F.Cu") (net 13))
 (segment (start 128.27 34.29) (end 113.03 34.29) (width 0.25) (layer "F.Cu") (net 13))
 (segment (start 113.03 34.29) (end 110.49 31.75) (width 0.25) (layer "F.Cu") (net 13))
 (segment (start 129.54 33.02) (end 128.27 34.29) (width 0.25) (layer "F.Cu") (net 13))
 (segment (start 110.49 31.75) (end 110.49 29.21) (width 0.25) (layer "F.Cu") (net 13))
 (segment (start 113.03 30.48) (end 113.03 29.21) (width 0.25) (layer "F.Cu") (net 14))
 (segment (start 135.89 30.48) (end 128.27 30.48) (width 0.25) (layer "F.Cu") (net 14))
 (segment (start 127 31.75) (end 114.3 31.75) (width 0.25) (layer "F.Cu") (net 14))
 (segment (start 128.27 30.48) (end 127 31.75) (width 0.25) (layer "F.Cu") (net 14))
 (segment (start 114.3 31.75) (end 113.03 30.48) (width 0.25) (layer "F.Cu") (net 14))
 (segment (start 125.73 29.21) (end 120.65 29.21) (width 0.25) (layer "F.Cu") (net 15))
 (segment (start 135.89 27.94) (end 127 27.94) (width 0.25) (layer "F.Cu") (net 15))
 (segment (start 127 27.94) (end 125.73 29.21) (width 0.25) (layer "F.Cu") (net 15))
 (segment (start 135.89 35.56) (end 111.76 35.56) (width 0.25) (layer "F.Cu") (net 12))
 (segment (start 111.76 35.56) (end 107.95 31.75) (width 0.25) (layer "F.Cu") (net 12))
 (segment (start 107.95 31.75) (end 107.95 29.21) (width 0.25) (layer "F.Cu") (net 12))
 (segment (start 110.49 41.91) (end 110.49 46.99) (width 0.25) (layer "B.Cu") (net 10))
 (segment (start 135.89 40.64) (end 111.76 40.64) (width 0.25) (layer "B.Cu") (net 10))
 (segment (start 111.76 40.64) (end 110.49 41.91) (width 0.25) (layer "B.Cu") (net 10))
 (segment (start 114.3 38.1) (end 113.03 39.37) (width 0.25) (layer "F.Cu") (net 11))
 (segment (start 135.89 38.1) (end 114.3 38.1) (width 0.25) (layer "F.Cu") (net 11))
 (segment (start 113.03 39.37) (end 113.03 46.99) (width 0.25) (layer "F.Cu") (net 11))
 (segment (start 74.93 46.99) (end 74.93 50.8) (width 0.5) (layer "F.Cu") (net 17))
 (segment (start 74.93 50.8) (end 72.39 53.34) (width 0.5) (layer "F.Cu") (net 17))
 (segment (start 77.47 53.34) (end 77.47 46.99) (width 0.5) (layer "F.Cu") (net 18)))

